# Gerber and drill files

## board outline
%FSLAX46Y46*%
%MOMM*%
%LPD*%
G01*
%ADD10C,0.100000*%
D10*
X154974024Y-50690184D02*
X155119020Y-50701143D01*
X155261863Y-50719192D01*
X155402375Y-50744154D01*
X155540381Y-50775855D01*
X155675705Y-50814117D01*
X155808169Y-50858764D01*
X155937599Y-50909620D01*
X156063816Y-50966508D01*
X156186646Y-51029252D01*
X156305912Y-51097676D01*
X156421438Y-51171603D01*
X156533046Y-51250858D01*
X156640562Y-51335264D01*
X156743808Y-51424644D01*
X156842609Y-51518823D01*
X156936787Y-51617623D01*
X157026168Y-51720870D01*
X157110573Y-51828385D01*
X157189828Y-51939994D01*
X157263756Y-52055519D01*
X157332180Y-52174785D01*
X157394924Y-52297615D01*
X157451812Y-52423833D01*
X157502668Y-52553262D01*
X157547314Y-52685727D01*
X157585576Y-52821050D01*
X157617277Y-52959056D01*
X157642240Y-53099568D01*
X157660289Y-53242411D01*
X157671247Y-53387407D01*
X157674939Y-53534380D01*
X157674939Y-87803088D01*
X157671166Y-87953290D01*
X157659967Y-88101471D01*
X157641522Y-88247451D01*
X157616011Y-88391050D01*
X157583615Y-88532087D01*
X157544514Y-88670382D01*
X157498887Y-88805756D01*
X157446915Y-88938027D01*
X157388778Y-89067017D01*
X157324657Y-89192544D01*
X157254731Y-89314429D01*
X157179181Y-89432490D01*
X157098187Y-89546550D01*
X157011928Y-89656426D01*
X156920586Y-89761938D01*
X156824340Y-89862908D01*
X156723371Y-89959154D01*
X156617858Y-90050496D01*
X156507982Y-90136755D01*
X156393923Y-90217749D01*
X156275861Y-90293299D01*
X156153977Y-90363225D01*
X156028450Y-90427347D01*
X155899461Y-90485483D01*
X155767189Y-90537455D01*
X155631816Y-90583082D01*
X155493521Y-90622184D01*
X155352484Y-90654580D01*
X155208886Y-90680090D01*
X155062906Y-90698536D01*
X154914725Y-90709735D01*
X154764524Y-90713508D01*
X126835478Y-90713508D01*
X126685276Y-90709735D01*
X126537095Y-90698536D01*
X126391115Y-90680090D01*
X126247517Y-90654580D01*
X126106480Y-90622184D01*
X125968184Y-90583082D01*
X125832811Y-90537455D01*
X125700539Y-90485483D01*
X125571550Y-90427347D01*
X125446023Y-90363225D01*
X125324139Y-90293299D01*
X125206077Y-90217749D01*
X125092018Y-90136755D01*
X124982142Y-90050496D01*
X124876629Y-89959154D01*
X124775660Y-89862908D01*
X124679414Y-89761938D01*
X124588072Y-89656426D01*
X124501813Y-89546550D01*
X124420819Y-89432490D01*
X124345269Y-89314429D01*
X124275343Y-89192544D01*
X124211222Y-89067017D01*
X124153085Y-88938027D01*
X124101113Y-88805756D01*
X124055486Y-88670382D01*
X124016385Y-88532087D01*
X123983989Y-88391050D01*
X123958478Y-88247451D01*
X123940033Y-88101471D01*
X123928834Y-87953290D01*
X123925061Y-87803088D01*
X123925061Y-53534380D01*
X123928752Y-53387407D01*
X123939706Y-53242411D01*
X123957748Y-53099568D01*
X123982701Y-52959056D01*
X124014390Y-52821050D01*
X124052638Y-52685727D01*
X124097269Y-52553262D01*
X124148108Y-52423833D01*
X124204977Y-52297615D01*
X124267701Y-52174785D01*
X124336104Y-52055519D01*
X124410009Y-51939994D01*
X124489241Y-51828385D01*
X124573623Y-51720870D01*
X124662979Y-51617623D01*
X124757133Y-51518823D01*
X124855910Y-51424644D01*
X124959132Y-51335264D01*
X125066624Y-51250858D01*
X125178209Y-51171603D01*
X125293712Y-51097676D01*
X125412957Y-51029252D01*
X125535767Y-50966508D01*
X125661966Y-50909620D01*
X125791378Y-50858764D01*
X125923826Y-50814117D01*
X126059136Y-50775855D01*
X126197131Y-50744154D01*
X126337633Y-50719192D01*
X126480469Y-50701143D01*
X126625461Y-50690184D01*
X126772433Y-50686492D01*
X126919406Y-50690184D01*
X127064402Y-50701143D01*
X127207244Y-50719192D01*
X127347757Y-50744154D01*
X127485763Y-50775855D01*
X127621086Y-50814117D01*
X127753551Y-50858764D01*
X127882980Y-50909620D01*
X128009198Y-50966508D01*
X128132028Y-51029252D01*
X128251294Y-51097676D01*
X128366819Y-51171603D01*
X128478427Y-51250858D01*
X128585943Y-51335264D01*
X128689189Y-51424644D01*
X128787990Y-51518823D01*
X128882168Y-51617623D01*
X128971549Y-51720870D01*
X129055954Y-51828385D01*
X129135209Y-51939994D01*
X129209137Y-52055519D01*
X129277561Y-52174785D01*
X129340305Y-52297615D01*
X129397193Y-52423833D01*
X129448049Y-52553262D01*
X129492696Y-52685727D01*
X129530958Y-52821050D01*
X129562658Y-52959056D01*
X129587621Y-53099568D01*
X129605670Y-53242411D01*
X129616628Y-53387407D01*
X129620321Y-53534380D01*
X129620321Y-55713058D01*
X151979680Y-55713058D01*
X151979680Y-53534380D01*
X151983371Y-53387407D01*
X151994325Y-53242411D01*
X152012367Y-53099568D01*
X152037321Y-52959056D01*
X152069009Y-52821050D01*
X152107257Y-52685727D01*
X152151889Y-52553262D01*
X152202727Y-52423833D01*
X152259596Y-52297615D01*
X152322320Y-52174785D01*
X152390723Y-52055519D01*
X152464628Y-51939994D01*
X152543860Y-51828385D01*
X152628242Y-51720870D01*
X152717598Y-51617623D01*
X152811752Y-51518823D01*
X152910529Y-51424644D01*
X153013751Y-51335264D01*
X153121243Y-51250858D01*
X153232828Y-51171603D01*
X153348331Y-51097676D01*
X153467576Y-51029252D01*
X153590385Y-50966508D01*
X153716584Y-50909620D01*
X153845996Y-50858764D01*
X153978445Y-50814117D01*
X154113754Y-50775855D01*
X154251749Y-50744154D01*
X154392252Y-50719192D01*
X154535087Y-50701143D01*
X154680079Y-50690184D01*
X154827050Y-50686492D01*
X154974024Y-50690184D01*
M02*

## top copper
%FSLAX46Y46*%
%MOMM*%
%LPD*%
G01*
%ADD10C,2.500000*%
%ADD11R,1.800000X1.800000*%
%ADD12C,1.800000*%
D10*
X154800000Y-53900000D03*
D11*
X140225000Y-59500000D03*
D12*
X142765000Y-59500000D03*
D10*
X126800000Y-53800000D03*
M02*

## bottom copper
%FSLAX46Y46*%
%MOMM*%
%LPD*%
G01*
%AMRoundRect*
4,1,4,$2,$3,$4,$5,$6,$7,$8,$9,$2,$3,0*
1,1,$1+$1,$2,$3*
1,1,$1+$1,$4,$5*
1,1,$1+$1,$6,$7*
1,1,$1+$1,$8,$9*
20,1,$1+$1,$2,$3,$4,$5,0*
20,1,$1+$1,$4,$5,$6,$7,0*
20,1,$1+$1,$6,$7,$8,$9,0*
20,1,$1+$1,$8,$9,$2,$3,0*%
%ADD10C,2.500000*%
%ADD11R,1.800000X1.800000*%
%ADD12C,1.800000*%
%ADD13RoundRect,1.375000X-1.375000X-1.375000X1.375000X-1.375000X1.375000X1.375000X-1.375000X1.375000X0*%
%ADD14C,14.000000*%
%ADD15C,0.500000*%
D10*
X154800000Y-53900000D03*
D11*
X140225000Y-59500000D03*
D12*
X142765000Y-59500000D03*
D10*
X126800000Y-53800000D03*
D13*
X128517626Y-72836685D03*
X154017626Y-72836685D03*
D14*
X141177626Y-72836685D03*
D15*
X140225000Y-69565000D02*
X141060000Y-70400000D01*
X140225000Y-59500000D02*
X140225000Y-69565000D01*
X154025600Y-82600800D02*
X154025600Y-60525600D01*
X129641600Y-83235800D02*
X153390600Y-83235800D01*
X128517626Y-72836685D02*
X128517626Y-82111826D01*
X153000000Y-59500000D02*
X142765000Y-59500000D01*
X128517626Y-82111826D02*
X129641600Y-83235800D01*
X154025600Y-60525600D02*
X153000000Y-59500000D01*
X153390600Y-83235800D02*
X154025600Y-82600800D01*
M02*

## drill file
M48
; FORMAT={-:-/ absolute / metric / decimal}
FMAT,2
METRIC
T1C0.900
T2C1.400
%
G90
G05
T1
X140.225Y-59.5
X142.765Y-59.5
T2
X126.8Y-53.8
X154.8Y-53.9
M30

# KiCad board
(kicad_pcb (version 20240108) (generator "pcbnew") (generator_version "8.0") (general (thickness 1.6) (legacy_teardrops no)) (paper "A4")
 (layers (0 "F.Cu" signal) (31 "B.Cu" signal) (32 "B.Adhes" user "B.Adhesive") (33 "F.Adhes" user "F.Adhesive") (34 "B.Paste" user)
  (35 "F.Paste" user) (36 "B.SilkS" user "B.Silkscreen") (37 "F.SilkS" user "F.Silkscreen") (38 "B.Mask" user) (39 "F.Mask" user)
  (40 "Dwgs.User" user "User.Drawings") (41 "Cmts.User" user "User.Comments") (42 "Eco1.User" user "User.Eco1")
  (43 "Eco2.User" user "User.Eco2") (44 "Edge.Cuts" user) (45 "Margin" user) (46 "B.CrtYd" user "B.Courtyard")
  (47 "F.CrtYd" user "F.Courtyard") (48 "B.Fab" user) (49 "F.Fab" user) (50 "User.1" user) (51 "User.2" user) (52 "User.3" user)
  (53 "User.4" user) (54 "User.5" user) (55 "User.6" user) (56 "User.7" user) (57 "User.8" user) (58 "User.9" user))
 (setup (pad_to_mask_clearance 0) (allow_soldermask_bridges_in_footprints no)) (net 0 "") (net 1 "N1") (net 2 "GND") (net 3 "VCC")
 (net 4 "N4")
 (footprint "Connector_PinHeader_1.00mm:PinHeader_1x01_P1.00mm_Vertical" (layer "F.Cu") (at 154.8 53.9)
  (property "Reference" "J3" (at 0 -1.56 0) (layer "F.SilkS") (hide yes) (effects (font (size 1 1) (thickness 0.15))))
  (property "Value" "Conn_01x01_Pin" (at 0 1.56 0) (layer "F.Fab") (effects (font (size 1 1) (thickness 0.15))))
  (pad "1" thru_hole circle (at 0 0) (size 2.5 2.5) (drill 1.4) (layers "*.Cu" "*.Mask") (remove_unused_layers no) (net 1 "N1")))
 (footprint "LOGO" (layer "F.Cu") (at 141.5 73)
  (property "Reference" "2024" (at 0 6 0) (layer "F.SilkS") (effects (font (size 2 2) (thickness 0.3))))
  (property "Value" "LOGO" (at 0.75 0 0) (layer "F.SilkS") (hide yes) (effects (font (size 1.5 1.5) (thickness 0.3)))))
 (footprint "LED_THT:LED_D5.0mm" (layer "F.Cu") (at 140.225 59.5)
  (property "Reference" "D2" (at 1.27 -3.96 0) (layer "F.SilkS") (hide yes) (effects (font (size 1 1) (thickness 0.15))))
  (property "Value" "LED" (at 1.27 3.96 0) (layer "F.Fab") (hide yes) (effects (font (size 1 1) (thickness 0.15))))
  (pad "1" thru_hole rect (at 0 0) (size 1.8 1.8) (drill 0.9) (layers "*.Cu" "*.Mask") (remove_unused_layers no) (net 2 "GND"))
  (pad "2" thru_hole circle (at 2.54 0) (size 1.8 1.8) (drill 0.9) (layers "*.Cu" "*.Mask") (remove_unused_layers no) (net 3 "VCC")))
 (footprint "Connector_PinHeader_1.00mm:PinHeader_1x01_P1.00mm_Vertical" (layer "F.Cu") (at 126.8 53.8)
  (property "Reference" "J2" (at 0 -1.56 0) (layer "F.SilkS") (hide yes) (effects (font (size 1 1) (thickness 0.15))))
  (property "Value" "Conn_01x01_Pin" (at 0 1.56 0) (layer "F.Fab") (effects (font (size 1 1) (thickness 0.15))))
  (pad "1" thru_hole circle (at 0 0) (size 2.5 2.5) (drill 1.4) (layers "*.Cu" "*.Mask") (remove_unused_layers no) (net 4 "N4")))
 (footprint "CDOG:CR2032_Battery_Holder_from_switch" (layer "F.Cu") (at 141.267626 72.836685)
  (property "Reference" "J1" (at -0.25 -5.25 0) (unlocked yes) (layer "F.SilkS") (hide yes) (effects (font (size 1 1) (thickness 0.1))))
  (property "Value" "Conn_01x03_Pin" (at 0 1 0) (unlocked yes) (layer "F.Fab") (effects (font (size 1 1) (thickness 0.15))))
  (pad "1" smd roundrect (at -12.75 0) (size 5.5 5.5) (layers "B.Cu" "B.Paste" "B.Mask") (roundrect_rratio 0.25) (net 3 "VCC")
   (thermal_bridge_angle 45))
  (pad "2" smd roundrect (at 12.75 0) (size 5.5 5.5) (layers "B.Cu" "B.Paste" "B.Mask") (roundrect_rratio 0.25) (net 3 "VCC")
   (thermal_bridge_angle 45))
  (pad "3" smd circle (at -0.09 0) (size 14 14) (layers "B.Cu" "B.Paste" "B.Mask") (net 2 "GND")))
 (gr_poly
  (pts (xy 154.974024 50.690184) (xy 155.11902 50.701143) (xy 155.261863 50.719192) (xy 155.402375 50.744154) (xy 155.540381 50.775855)
   (xy 155.675705 50.814117) (xy 155.808169 50.858764) (xy 155.937599 50.90962) (xy 156.063816 50.966508) (xy 156.186646 51.029252)
   (xy 156.305912 51.097676) (xy 156.421438 51.171603) (xy 156.533046 51.250858) (xy 156.640562 51.335264) (xy 156.743808 51.424644)
   (xy 156.842609 51.518823) (xy 156.936787 51.617623) (xy 157.026168 51.72087) (xy 157.110573 51.828385) (xy 157.189828 51.939994)
   (xy 157.263756 52.055519) (xy 157.33218 52.174785) (xy 157.394924 52.297615) (xy 157.451812 52.423833) (xy 157.502668 52.553262)
   (xy 157.547314 52.685727) (xy 157.585576 52.82105) (xy 157.617277 52.959056) (xy 157.64224 53.099568) (xy 157.660289 53.242411)
   (xy 157.671247 53.387407) (xy 157.674939 53.53438) (xy 157.674939 87.803088) (xy 157.671166 87.95329) (xy 157.659967 88.101471)
   (xy 157.641522 88.247451) (xy 157.616011 88.39105) (xy 157.583615 88.532087) (xy 157.544514 88.670382) (xy 157.498887 88.805756)
   (xy 157.446915 88.938027) (xy 157.388778 89.067017) (xy 157.324657 89.192544) (xy 157.254731 89.314429) (xy 157.179181 89.43249)
   (xy 157.098187 89.54655) (xy 157.011928 89.656426) (xy 156.920586 89.761938) (xy 156.82434 89.862908) (xy 156.723371 89.959154)
   (xy 156.617858 90.050496) (xy 156.507982 90.136755) (xy 156.393923 90.217749) (xy 156.275861 90.293299) (xy 156.153977 90.363225)
   (xy 156.02845 90.427347) (xy 155.899461 90.485483) (xy 155.767189 90.537455) (xy 155.631816 90.583082) (xy 155.493521 90.622184)
   (xy 155.352484 90.65458) (xy 155.208886 90.68009) (xy 155.062906 90.698536) (xy 154.914725 90.709735) (xy 154.764524 90.713508)
   (xy 126.835478 90.713508) (xy 126.685276 90.709735) (xy 126.537095 90.698536) (xy 126.391115 90.68009) (xy 126.247517 90.65458)
   (xy 126.10648 90.622184) (xy 125.968184 90.583082) (xy 125.832811 90.537455) (xy 125.700539 90.485483) (xy 125.57155 90.427347)
   (xy 125.446023 90.363225) (xy 125.324139 90.293299) (xy 125.206077 90.217749) (xy 125.092018 90.136755) (xy 124.982142 90.050496)
   (xy 124.876629 89.959154) (xy 124.77566 89.862908) (xy 124.679414 89.761938) (xy 124.588072 89.656426) (xy 124.501813 89.54655)
   (xy 124.420819 89.43249) (xy 124.345269 89.314429) (xy 124.275343 89.192544) (xy 124.211222 89.067017) (xy 124.153085 88.938027)
   (xy 124.101113 88.805756) (xy 124.055486 88.670382) (xy 124.016385 88.532087) (xy 123.983989 88.39105) (xy 123.958478 88.247451)
   (xy 123.940033 88.101471) (xy 123.928834 87.95329) (xy 123.925061 87.803088) (xy 123.925061 53.53438) (xy 123.928752 53.387407)
   (xy 123.939706 53.242411) (xy 123.957748 53.099568) (xy 123.982701 52.959056) (xy 124.01439 52.82105) (xy 124.052638 52.685727)
   (xy 124.097269 52.553262) (xy 124.148108 52.423833) (xy 124.204977 52.297615) (xy 124.267701 52.174785) (xy 124.336104 52.055519)
   (xy 124.410009 51.939994) (xy 124.489241 51.828385) (xy 124.573623 51.72087) (xy 124.662979 51.617623) (xy 124.757133 51.518823)
   (xy 124.85591 51.424644) (xy 124.959132 51.335264) (xy 125.066624 51.250858) (xy 125.178209 51.171603) (xy 125.293712 51.097676)
   (xy 125.412957 51.029252) (xy 125.535767 50.966508) (xy 125.661966 50.90962) (xy 125.791378 50.858764) (xy 125.923826 50.814117)
   (xy 126.059136 50.775855) (xy 126.197131 50.744154) (xy 126.337633 50.719192) (xy 126.480469 50.701143) (xy 126.625461 50.690184)
   (xy 126.772433 50.686492) (xy 126.919406 50.690184) (xy 127.064402 50.701143) (xy 127.207244 50.719192) (xy 127.347757 50.744154)
   (xy 127.485763 50.775855) (xy 127.621086 50.814117) (xy 127.753551 50.858764) (xy 127.88298 50.90962) (xy 128.009198 50.966508)
   (xy 128.132028 51.029252) (xy 128.251294 51.097676) (xy 128.366819 51.171603) (xy 128.478427 51.250858) (xy 128.585943 51.335264)
   (xy 128.689189 51.424644) (xy 128.78799 51.518823) (xy 128.882168 51.617623) (xy 128.971549 51.72087) (xy 129.055954 51.828385)
   (xy 129.135209 51.939994) (xy 129.209137 52.055519) (xy 129.277561 52.174785) (xy 129.340305 52.297615) (xy 129.397193 52.423833)
   (xy 129.448049 52.553262) (xy 129.492696 52.685727) (xy 129.530958 52.82105) (xy 129.562658 52.959056) (xy 129.587621 53.099568)
   (xy 129.60567 53.242411) (xy 129.616628 53.387407) (xy 129.620321 53.53438) (xy 129.620321 55.713058) (xy 151.97968 55.713058)
   (xy 151.97968 53.53438) (xy 151.983371 53.387407) (xy 151.994325 53.242411) (xy 152.012367 53.099568) (xy 152.037321 52.959056)
   (xy 152.069009 52.82105) (xy 152.107257 52.685727) (xy 152.151889 52.553262) (xy 152.202727 52.423833) (xy 152.259596 52.297615)
   (xy 152.32232 52.174785) (xy 152.390723 52.055519) (xy 152.464628 51.939994) (xy 152.54386 51.828385) (xy 152.628242 51.72087)
   (xy 152.717598 51.617623) (xy 152.811752 51.518823) (xy 152.910529 51.424644) (xy 153.013751 51.335264) (xy 153.121243 51.250858)
   (xy 153.232828 51.171603) (xy 153.348331 51.097676) (xy 153.467576 51.029252) (xy 153.590385 50.966508) (xy 153.716584 50.90962)
   (xy 153.845996 50.858764) (xy 153.978445 50.814117) (xy 154.113754 50.775855) (xy 154.251749 50.744154) (xy 154.392252 50.719192)
   (xy 154.535087 50.701143) (xy 154.680079 50.690184) (xy 154.82705 50.686492))
  (stroke (width 0.1) (type solid) (color 155 141 141 1)) (fill none) (layer "Edge.Cuts"))
 (segment (start 140.225 69.565) (end 141.06 70.4) (width 0.5) (layer "B.Cu") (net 2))
 (segment (start 140.225 59.5) (end 140.225 69.565) (width 0.5) (layer "B.Cu") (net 2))
 (segment (start 154.0256 82.6008) (end 154.0256 60.5256) (width 0.5) (layer "B.Cu") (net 3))
 (segment (start 129.6416 83.2358) (end 153.3906 83.2358) (width 0.5) (layer "B.Cu") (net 3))
 (segment (start 128.517626 72.836685) (end 128.517626 82.111826) (width 0.5) (layer "B.Cu") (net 3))
 (segment (start 153 59.5) (end 142.765 59.5) (width 0.5) (layer "B.Cu") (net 3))
 (segment (start 128.517626 82.111826) (end 129.6416 83.2358) (width 0.5) (layer "B.Cu") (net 3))
 (segment (start 154.0256 60.5256) (end 153 59.5) (width 0.5) (layer "B.Cu") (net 3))
 (segment (start 153.3906 83.2358) (end 154.0256 82.6008) (width 0.5) (layer "B.Cu") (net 3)))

